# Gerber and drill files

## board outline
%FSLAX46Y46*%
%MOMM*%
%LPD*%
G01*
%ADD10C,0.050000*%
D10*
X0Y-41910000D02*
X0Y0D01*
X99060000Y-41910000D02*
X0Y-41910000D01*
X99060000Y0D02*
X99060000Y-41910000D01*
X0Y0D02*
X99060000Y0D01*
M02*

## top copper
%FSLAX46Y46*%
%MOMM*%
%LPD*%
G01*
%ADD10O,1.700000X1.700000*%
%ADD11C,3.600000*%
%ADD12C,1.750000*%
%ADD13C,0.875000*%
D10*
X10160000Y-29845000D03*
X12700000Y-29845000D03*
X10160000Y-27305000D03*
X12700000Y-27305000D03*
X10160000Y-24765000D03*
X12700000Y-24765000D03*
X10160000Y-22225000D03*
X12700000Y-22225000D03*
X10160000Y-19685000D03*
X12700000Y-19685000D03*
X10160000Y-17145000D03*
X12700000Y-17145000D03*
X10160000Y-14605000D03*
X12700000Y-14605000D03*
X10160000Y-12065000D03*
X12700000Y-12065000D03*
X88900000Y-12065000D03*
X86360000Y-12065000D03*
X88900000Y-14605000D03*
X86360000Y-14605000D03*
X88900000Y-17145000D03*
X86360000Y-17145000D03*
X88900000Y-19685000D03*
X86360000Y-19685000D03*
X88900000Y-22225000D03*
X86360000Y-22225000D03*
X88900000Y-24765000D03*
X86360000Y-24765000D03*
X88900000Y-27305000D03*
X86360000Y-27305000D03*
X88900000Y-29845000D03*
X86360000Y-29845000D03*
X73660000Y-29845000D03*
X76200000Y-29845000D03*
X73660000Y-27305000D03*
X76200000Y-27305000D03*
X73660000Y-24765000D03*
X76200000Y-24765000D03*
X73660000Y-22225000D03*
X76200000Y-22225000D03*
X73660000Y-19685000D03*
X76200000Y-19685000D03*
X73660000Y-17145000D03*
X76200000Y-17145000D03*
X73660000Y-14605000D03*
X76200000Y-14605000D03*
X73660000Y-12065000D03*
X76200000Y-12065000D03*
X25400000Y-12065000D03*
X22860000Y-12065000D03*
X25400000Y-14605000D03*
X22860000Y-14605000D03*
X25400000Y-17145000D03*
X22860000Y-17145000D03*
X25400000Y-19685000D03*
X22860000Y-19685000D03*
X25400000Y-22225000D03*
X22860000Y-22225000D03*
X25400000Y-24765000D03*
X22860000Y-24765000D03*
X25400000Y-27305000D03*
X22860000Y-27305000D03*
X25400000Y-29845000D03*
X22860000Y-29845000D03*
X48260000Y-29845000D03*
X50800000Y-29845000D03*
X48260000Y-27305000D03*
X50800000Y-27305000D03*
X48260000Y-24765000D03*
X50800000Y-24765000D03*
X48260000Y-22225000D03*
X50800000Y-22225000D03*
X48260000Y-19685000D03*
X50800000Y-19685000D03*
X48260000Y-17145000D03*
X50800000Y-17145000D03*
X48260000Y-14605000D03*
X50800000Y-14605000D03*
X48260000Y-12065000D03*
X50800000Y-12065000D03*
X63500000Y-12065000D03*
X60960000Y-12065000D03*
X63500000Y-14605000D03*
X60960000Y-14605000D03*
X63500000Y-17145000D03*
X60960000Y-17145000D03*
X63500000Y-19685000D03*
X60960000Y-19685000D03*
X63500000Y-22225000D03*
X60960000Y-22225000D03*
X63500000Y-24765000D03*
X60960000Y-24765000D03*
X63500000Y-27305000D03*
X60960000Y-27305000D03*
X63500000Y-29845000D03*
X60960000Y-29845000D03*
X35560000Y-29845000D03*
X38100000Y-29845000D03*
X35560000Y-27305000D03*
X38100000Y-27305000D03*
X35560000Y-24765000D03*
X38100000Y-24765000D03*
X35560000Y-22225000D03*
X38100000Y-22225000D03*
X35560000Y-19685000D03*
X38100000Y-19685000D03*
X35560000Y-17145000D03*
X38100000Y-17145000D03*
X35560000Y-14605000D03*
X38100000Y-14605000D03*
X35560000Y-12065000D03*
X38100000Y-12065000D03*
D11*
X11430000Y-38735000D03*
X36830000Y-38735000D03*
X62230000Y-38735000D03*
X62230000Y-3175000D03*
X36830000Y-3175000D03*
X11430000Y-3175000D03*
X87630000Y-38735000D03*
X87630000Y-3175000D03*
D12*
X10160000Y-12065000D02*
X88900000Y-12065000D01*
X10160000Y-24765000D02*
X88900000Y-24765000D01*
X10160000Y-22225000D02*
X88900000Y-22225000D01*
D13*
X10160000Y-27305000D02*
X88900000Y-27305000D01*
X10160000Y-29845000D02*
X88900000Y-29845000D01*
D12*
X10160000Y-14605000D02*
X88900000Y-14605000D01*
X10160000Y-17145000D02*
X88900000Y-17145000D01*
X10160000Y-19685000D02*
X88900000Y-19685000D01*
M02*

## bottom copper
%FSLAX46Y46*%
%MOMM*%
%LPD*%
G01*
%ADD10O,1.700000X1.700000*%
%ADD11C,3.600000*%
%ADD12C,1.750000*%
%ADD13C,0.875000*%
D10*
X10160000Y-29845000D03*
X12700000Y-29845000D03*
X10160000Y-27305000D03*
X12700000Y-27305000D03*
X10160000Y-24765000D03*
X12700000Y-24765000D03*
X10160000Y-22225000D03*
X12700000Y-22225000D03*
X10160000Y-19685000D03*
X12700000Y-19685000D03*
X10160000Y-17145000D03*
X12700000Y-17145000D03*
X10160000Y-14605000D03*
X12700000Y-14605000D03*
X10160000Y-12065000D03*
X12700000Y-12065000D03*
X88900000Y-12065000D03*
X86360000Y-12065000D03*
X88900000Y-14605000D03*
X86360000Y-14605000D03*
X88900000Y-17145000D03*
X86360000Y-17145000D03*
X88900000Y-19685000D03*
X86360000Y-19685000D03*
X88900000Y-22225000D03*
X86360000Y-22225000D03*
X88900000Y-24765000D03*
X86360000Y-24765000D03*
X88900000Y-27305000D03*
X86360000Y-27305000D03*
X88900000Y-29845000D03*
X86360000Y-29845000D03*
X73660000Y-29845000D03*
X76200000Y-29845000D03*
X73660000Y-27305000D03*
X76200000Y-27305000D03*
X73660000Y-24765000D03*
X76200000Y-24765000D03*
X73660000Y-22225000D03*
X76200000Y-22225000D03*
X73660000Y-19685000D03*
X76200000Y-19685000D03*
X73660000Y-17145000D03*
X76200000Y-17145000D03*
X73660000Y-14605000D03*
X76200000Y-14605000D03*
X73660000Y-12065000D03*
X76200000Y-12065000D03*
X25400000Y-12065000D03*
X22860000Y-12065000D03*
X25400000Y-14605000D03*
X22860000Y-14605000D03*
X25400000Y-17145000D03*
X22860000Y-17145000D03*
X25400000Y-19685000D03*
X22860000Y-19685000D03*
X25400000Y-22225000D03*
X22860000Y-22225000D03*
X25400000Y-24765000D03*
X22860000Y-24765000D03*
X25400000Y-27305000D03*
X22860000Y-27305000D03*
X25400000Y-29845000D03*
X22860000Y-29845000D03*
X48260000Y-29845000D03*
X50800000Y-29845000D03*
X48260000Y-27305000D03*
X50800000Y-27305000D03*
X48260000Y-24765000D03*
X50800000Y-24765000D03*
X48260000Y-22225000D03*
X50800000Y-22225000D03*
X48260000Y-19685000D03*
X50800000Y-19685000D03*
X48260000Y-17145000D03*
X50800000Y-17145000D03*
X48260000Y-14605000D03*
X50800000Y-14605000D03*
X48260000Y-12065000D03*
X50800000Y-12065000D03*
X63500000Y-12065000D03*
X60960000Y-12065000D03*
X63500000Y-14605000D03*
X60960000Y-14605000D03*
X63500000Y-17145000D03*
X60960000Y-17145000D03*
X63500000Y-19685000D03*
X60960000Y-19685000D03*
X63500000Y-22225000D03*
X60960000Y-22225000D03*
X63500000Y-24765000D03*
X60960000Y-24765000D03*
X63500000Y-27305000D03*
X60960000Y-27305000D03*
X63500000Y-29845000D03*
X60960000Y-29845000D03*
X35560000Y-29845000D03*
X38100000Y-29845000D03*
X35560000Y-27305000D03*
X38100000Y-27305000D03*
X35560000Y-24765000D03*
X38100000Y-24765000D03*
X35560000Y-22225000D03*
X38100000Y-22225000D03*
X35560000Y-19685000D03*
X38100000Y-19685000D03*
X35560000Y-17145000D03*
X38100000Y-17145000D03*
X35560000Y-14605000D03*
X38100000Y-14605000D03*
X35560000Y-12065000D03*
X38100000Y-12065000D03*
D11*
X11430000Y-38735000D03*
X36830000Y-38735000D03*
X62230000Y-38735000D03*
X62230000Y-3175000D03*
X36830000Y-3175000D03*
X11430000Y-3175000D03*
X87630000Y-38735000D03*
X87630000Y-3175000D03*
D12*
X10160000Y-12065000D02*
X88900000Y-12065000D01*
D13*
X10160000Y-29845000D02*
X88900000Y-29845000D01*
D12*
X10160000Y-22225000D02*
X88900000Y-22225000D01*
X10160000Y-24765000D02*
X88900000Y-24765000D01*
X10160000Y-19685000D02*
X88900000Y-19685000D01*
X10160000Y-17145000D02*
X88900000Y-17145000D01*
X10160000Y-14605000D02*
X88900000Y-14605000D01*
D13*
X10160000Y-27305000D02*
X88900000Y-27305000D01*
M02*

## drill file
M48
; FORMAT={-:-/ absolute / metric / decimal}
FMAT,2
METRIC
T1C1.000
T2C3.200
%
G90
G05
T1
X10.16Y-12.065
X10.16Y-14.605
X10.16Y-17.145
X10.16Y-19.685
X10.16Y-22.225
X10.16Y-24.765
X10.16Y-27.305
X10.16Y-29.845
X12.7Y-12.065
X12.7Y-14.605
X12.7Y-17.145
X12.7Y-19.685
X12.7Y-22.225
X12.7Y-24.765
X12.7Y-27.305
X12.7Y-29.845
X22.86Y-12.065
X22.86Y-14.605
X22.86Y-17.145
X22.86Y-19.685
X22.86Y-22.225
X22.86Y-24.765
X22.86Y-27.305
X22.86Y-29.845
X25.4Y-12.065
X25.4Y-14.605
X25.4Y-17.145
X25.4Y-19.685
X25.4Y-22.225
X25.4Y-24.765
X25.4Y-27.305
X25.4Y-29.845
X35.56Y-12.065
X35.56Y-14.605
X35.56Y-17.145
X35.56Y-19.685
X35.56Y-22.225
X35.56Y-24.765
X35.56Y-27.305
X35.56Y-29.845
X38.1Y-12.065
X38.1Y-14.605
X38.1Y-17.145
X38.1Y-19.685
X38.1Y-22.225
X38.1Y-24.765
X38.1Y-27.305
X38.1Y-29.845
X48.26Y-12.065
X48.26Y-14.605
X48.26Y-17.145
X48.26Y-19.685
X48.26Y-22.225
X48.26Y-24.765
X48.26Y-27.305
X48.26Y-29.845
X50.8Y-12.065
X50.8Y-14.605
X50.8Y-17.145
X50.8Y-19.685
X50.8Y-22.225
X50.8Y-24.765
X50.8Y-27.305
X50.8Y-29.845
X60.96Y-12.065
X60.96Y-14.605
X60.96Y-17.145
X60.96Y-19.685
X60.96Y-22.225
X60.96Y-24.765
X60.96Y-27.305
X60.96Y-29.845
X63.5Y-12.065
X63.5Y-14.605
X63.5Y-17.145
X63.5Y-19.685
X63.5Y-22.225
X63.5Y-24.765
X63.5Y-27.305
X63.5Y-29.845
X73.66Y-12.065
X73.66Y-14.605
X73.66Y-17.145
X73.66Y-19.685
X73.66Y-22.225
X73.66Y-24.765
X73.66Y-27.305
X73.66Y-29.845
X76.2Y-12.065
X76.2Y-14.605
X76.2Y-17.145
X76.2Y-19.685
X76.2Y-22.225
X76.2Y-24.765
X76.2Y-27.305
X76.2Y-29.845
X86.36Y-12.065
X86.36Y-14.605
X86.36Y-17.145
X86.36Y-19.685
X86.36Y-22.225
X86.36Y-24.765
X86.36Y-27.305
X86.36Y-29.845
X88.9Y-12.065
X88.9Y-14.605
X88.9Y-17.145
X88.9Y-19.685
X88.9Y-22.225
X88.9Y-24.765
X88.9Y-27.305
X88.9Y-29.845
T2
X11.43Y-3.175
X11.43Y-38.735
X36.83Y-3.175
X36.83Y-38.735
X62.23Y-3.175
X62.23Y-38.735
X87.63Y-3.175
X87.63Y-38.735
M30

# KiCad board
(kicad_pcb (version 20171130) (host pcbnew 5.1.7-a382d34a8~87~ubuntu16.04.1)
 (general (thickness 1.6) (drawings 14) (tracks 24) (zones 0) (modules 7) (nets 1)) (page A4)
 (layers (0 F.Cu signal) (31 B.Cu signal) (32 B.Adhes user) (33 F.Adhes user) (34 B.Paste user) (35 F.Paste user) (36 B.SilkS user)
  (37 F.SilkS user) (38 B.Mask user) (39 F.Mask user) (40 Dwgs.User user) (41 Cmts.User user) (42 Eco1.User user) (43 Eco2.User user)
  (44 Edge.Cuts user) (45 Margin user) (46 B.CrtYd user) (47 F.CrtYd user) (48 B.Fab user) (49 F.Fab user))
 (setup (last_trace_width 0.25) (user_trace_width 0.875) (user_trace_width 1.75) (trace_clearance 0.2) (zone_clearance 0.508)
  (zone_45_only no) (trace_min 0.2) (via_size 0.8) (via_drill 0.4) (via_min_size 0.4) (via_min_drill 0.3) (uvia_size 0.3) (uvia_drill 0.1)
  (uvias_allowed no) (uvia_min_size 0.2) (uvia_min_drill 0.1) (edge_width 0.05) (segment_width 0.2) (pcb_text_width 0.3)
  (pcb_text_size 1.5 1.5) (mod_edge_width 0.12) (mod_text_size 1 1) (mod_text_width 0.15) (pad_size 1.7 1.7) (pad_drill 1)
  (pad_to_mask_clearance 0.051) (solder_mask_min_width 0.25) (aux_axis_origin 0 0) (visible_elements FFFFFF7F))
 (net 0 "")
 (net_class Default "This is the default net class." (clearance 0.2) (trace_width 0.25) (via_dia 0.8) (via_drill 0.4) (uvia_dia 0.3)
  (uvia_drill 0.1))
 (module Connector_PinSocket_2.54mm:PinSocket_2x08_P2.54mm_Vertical (layer F.Cu) (at 12.7 12.065)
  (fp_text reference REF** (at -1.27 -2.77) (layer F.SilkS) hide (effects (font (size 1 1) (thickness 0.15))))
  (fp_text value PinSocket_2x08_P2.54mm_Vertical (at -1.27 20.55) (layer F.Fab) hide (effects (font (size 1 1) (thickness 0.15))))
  (pad 16 thru_hole oval (at -2.54 17.78) (size 1.7 1.7) (drill 1) (layers *.Cu *.Mask))
  (pad 15 thru_hole oval (at 0 17.78) (size 1.7 1.7) (drill 1) (layers *.Cu *.Mask))
  (pad 14 thru_hole oval (at -2.54 15.24) (size 1.7 1.7) (drill 1) (layers *.Cu *.Mask))
  (pad 13 thru_hole oval (at 0 15.24) (size 1.7 1.7) (drill 1) (layers *.Cu *.Mask))
  (pad 12 thru_hole oval (at -2.54 12.7) (size 1.7 1.7) (drill 1) (layers *.Cu *.Mask))
  (pad 11 thru_hole oval (at 0 12.7) (size 1.7 1.7) (drill 1) (layers *.Cu *.Mask))
  (pad 10 thru_hole oval (at -2.54 10.16) (size 1.7 1.7) (drill 1) (layers *.Cu *.Mask))
  (pad 9 thru_hole oval (at 0 10.16) (size 1.7 1.7) (drill 1) (layers *.Cu *.Mask))
  (pad 8 thru_hole oval (at -2.54 7.62) (size 1.7 1.7) (drill 1) (layers *.Cu *.Mask))
  (pad 7 thru_hole oval (at 0 7.62) (size 1.7 1.7) (drill 1) (layers *.Cu *.Mask))
  (pad 6 thru_hole oval (at -2.54 5.08) (size 1.7 1.7) (drill 1) (layers *.Cu *.Mask))
  (pad 5 thru_hole oval (at 0 5.08) (size 1.7 1.7) (drill 1) (layers *.Cu *.Mask))
  (pad 4 thru_hole oval (at -2.54 2.54) (size 1.7 1.7) (drill 1) (layers *.Cu *.Mask))
  (pad 3 thru_hole oval (at 0 2.54) (size 1.7 1.7) (drill 1) (layers *.Cu *.Mask))
  (pad 2 thru_hole oval (at -2.54 0) (size 1.7 1.7) (drill 1) (layers *.Cu *.Mask))
  (pad 1 thru_hole oval (at 0 0) (size 1.7 1.7) (drill 1) (layers *.Cu *.Mask)))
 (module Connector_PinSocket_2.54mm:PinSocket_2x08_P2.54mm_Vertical (layer F.Cu) (at 88.9 12.065)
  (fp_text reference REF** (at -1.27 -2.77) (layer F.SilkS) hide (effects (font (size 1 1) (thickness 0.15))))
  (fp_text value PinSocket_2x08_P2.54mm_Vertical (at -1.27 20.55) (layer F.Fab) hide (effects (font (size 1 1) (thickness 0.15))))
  (pad 1 thru_hole oval (at 0 0) (size 1.7 1.7) (drill 1) (layers *.Cu *.Mask))
  (pad 2 thru_hole oval (at -2.54 0) (size 1.7 1.7) (drill 1) (layers *.Cu *.Mask))
  (pad 3 thru_hole oval (at 0 2.54) (size 1.7 1.7) (drill 1) (layers *.Cu *.Mask))
  (pad 4 thru_hole oval (at -2.54 2.54) (size 1.7 1.7) (drill 1) (layers *.Cu *.Mask))
  (pad 5 thru_hole oval (at 0 5.08) (size 1.7 1.7) (drill 1) (layers *.Cu *.Mask))
  (pad 6 thru_hole oval (at -2.54 5.08) (size 1.7 1.7) (drill 1) (layers *.Cu *.Mask))
  (pad 7 thru_hole oval (at 0 7.62) (size 1.7 1.7) (drill 1) (layers *.Cu *.Mask))
  (pad 8 thru_hole oval (at -2.54 7.62) (size 1.7 1.7) (drill 1) (layers *.Cu *.Mask))
  (pad 9 thru_hole oval (at 0 10.16) (size 1.7 1.7) (drill 1) (layers *.Cu *.Mask))
  (pad 10 thru_hole oval (at -2.54 10.16) (size 1.7 1.7) (drill 1) (layers *.Cu *.Mask))
  (pad 11 thru_hole oval (at 0 12.7) (size 1.7 1.7) (drill 1) (layers *.Cu *.Mask))
  (pad 12 thru_hole oval (at -2.54 12.7) (size 1.7 1.7) (drill 1) (layers *.Cu *.Mask))
  (pad 13 thru_hole oval (at 0 15.24) (size 1.7 1.7) (drill 1) (layers *.Cu *.Mask))
  (pad 14 thru_hole oval (at -2.54 15.24) (size 1.7 1.7) (drill 1) (layers *.Cu *.Mask))
  (pad 15 thru_hole oval (at 0 17.78) (size 1.7 1.7) (drill 1) (layers *.Cu *.Mask))
  (pad 16 thru_hole oval (at -2.54 17.78) (size 1.7 1.7) (drill 1) (layers *.Cu *.Mask)))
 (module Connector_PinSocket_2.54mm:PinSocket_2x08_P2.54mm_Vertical (layer F.Cu) (at 76.2 12.065)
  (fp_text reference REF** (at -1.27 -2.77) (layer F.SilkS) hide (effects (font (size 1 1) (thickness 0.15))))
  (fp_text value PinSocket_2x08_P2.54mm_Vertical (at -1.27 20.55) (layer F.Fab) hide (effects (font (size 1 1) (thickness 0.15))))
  (pad 16 thru_hole oval (at -2.54 17.78) (size 1.7 1.7) (drill 1) (layers *.Cu *.Mask))
  (pad 15 thru_hole oval (at 0 17.78) (size 1.7 1.7) (drill 1) (layers *.Cu *.Mask))
  (pad 14 thru_hole oval (at -2.54 15.24) (size 1.7 1.7) (drill 1) (layers *.Cu *.Mask))
  (pad 13 thru_hole oval (at 0 15.24) (size 1.7 1.7) (drill 1) (layers *.Cu *.Mask))
  (pad 12 thru_hole oval (at -2.54 12.7) (size 1.7 1.7) (drill 1) (layers *.Cu *.Mask))
  (pad 11 thru_hole oval (at 0 12.7) (size 1.7 1.7) (drill 1) (layers *.Cu *.Mask))
  (pad 10 thru_hole oval (at -2.54 10.16) (size 1.7 1.7) (drill 1) (layers *.Cu *.Mask))
  (pad 9 thru_hole oval (at 0 10.16) (size 1.7 1.7) (drill 1) (layers *.Cu *.Mask))
  (pad 8 thru_hole oval (at -2.54 7.62) (size 1.7 1.7) (drill 1) (layers *.Cu *.Mask))
  (pad 7 thru_hole oval (at 0 7.62) (size 1.7 1.7) (drill 1) (layers *.Cu *.Mask))
  (pad 6 thru_hole oval (at -2.54 5.08) (size 1.7 1.7) (drill 1) (layers *.Cu *.Mask))
  (pad 5 thru_hole oval (at 0 5.08) (size 1.7 1.7) (drill 1) (layers *.Cu *.Mask))
  (pad 4 thru_hole oval (at -2.54 2.54) (size 1.7 1.7) (drill 1) (layers *.Cu *.Mask))
  (pad 3 thru_hole oval (at 0 2.54) (size 1.7 1.7) (drill 1) (layers *.Cu *.Mask))
  (pad 2 thru_hole oval (at -2.54 0) (size 1.7 1.7) (drill 1) (layers *.Cu *.Mask))
  (pad 1 thru_hole oval (at 0 0) (size 1.7 1.7) (drill 1) (layers *.Cu *.Mask)))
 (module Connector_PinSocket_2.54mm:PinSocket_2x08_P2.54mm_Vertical (layer F.Cu) (at 25.4 12.065)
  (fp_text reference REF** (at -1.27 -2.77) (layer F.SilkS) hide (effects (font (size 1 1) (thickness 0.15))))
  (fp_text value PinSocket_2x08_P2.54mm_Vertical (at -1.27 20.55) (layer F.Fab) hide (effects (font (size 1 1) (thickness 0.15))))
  (pad 1 thru_hole oval (at 0 0) (size 1.7 1.7) (drill 1) (layers *.Cu *.Mask))
  (pad 2 thru_hole oval (at -2.54 0) (size 1.7 1.7) (drill 1) (layers *.Cu *.Mask))
  (pad 3 thru_hole oval (at 0 2.54) (size 1.7 1.7) (drill 1) (layers *.Cu *.Mask))
  (pad 4 thru_hole oval (at -2.54 2.54) (size 1.7 1.7) (drill 1) (layers *.Cu *.Mask))
  (pad 5 thru_hole oval (at 0 5.08) (size 1.7 1.7) (drill 1) (layers *.Cu *.Mask))
  (pad 6 thru_hole oval (at -2.54 5.08) (size 1.7 1.7) (drill 1) (layers *.Cu *.Mask))
  (pad 7 thru_hole oval (at 0 7.62) (size 1.7 1.7) (drill 1) (layers *.Cu *.Mask))
  (pad 8 thru_hole oval (at -2.54 7.62) (size 1.7 1.7) (drill 1) (layers *.Cu *.Mask))
  (pad 9 thru_hole oval (at 0 10.16) (size 1.7 1.7) (drill 1) (layers *.Cu *.Mask))
  (pad 10 thru_hole oval (at -2.54 10.16) (size 1.7 1.7) (drill 1) (layers *.Cu *.Mask))
  (pad 11 thru_hole oval (at 0 12.7) (size 1.7 1.7) (drill 1) (layers *.Cu *.Mask))
  (pad 12 thru_hole oval (at -2.54 12.7) (size 1.7 1.7) (drill 1) (layers *.Cu *.Mask))
  (pad 13 thru_hole oval (at 0 15.24) (size 1.7 1.7) (drill 1) (layers *.Cu *.Mask))
  (pad 14 thru_hole oval (at -2.54 15.24) (size 1.7 1.7) (drill 1) (layers *.Cu *.Mask))
  (pad 15 thru_hole oval (at 0 17.78) (size 1.7 1.7) (drill 1) (layers *.Cu *.Mask))
  (pad 16 thru_hole oval (at -2.54 17.78) (size 1.7 1.7) (drill 1) (layers *.Cu *.Mask)))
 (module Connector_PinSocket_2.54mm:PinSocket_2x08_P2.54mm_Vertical (layer F.Cu) (at 50.8 12.065)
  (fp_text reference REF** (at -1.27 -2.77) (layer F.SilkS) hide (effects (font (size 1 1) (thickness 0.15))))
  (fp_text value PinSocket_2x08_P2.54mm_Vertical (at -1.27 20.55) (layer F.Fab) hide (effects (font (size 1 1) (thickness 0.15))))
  (pad 16 thru_hole oval (at -2.54 17.78) (size 1.7 1.7) (drill 1) (layers *.Cu *.Mask))
  (pad 15 thru_hole oval (at 0 17.78) (size 1.7 1.7) (drill 1) (layers *.Cu *.Mask))
  (pad 14 thru_hole oval (at -2.54 15.24) (size 1.7 1.7) (drill 1) (layers *.Cu *.Mask))
  (pad 13 thru_hole oval (at 0 15.24) (size 1.7 1.7) (drill 1) (layers *.Cu *.Mask))
  (pad 12 thru_hole oval (at -2.54 12.7) (size 1.7 1.7) (drill 1) (layers *.Cu *.Mask))
  (pad 11 thru_hole oval (at 0 12.7) (size 1.7 1.7) (drill 1) (layers *.Cu *.Mask))
  (pad 10 thru_hole oval (at -2.54 10.16) (size 1.7 1.7) (drill 1) (layers *.Cu *.Mask))
  (pad 9 thru_hole oval (at 0 10.16) (size 1.7 1.7) (drill 1) (layers *.Cu *.Mask))
  (pad 8 thru_hole oval (at -2.54 7.62) (size 1.7 1.7) (drill 1) (layers *.Cu *.Mask))
  (pad 7 thru_hole oval (at 0 7.62) (size 1.7 1.7) (drill 1) (layers *.Cu *.Mask))
  (pad 6 thru_hole oval (at -2.54 5.08) (size 1.7 1.7) (drill 1) (layers *.Cu *.Mask))
  (pad 5 thru_hole oval (at 0 5.08) (size 1.7 1.7) (drill 1) (layers *.Cu *.Mask))
  (pad 4 thru_hole oval (at -2.54 2.54) (size 1.7 1.7) (drill 1) (layers *.Cu *.Mask))
  (pad 3 thru_hole oval (at 0 2.54) (size 1.7 1.7) (drill 1) (layers *.Cu *.Mask))
  (pad 2 thru_hole oval (at -2.54 0) (size 1.7 1.7) (drill 1) (layers *.Cu *.Mask))
  (pad 1 thru_hole oval (at 0 0) (size 1.7 1.7) (drill 1) (layers *.Cu *.Mask)))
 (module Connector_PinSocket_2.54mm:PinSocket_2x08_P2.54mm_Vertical (layer F.Cu) (at 63.5 12.065)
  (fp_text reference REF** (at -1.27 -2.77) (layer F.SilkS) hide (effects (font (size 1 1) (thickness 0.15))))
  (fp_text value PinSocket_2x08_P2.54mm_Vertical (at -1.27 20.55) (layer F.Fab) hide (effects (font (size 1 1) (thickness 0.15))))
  (pad 1 thru_hole oval (at 0 0) (size 1.7 1.7) (drill 1) (layers *.Cu *.Mask))
  (pad 2 thru_hole oval (at -2.54 0) (size 1.7 1.7) (drill 1) (layers *.Cu *.Mask))
  (pad 3 thru_hole oval (at 0 2.54) (size 1.7 1.7) (drill 1) (layers *.Cu *.Mask))
  (pad 4 thru_hole oval (at -2.54 2.54) (size 1.7 1.7) (drill 1) (layers *.Cu *.Mask))
  (pad 5 thru_hole oval (at 0 5.08) (size 1.7 1.7) (drill 1) (layers *.Cu *.Mask))
  (pad 6 thru_hole oval (at -2.54 5.08) (size 1.7 1.7) (drill 1) (layers *.Cu *.Mask))
  (pad 7 thru_hole oval (at 0 7.62) (size 1.7 1.7) (drill 1) (layers *.Cu *.Mask))
  (pad 8 thru_hole oval (at -2.54 7.62) (size 1.7 1.7) (drill 1) (layers *.Cu *.Mask))
  (pad 9 thru_hole oval (at 0 10.16) (size 1.7 1.7) (drill 1) (layers *.Cu *.Mask))
  (pad 10 thru_hole oval (at -2.54 10.16) (size 1.7 1.7) (drill 1) (layers *.Cu *.Mask))
  (pad 11 thru_hole oval (at 0 12.7) (size 1.7 1.7) (drill 1) (layers *.Cu *.Mask))
  (pad 12 thru_hole oval (at -2.54 12.7) (size 1.7 1.7) (drill 1) (layers *.Cu *.Mask))
  (pad 13 thru_hole oval (at 0 15.24) (size 1.7 1.7) (drill 1) (layers *.Cu *.Mask))
  (pad 14 thru_hole oval (at -2.54 15.24) (size 1.7 1.7) (drill 1) (layers *.Cu *.Mask))
  (pad 15 thru_hole oval (at 0 17.78) (size 1.7 1.7) (drill 1) (layers *.Cu *.Mask))
  (pad 16 thru_hole oval (at -2.54 17.78) (size 1.7 1.7) (drill 1) (layers *.Cu *.Mask)))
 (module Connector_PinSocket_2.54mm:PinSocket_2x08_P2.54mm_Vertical (layer F.Cu) (at 38.1 12.065)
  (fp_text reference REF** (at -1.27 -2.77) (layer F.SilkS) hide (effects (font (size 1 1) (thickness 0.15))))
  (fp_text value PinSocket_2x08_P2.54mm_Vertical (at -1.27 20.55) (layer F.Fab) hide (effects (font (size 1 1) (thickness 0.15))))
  (pad 16 thru_hole oval (at -2.54 17.78) (size 1.7 1.7) (drill 1) (layers *.Cu *.Mask))
  (pad 15 thru_hole oval (at 0 17.78) (size 1.7 1.7) (drill 1) (layers *.Cu *.Mask))
  (pad 14 thru_hole oval (at -2.54 15.24) (size 1.7 1.7) (drill 1) (layers *.Cu *.Mask))
  (pad 13 thru_hole oval (at 0 15.24) (size 1.7 1.7) (drill 1) (layers *.Cu *.Mask))
  (pad 12 thru_hole oval (at -2.54 12.7) (size 1.7 1.7) (drill 1) (layers *.Cu *.Mask))
  (pad 11 thru_hole oval (at 0 12.7) (size 1.7 1.7) (drill 1) (layers *.Cu *.Mask))
  (pad 10 thru_hole oval (at -2.54 10.16) (size 1.7 1.7) (drill 1) (layers *.Cu *.Mask))
  (pad 9 thru_hole oval (at 0 10.16) (size 1.7 1.7) (drill 1) (layers *.Cu *.Mask))
  (pad 8 thru_hole oval (at -2.54 7.62) (size 1.7 1.7) (drill 1) (layers *.Cu *.Mask))
  (pad 7 thru_hole oval (at 0 7.62) (size 1.7 1.7) (drill 1) (layers *.Cu *.Mask))
  (pad 6 thru_hole oval (at -2.54 5.08) (size 1.7 1.7) (drill 1) (layers *.Cu *.Mask))
  (pad 5 thru_hole oval (at 0 5.08) (size 1.7 1.7) (drill 1) (layers *.Cu *.Mask))
  (pad 4 thru_hole oval (at -2.54 2.54) (size 1.7 1.7) (drill 1) (layers *.Cu *.Mask))
  (pad 3 thru_hole oval (at 0 2.54) (size 1.7 1.7) (drill 1) (layers *.Cu *.Mask))
  (pad 2 thru_hole oval (at -2.54 0) (size 1.7 1.7) (drill 1) (layers *.Cu *.Mask))
  (pad 1 thru_hole oval (at 0 0) (size 1.7 1.7) (drill 1) (layers *.Cu *.Mask)))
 (gr_line (start 0 41.91) (end 0 0) (layer Edge.Cuts) (width 0.05))
 (gr_line (start 99.06 41.91) (end 0 41.91) (layer Edge.Cuts) (width 0.05))
 (gr_line (start 99.06 0) (end 99.06 41.91) (layer Edge.Cuts) (width 0.05))
 (gr_line (start 0 0) (end 99.06 0) (layer Edge.Cuts) (width 0.05))
 (via (at 11.43 38.735) (size 3.6) (drill 3.2) (layers F.Cu B.Cu) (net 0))
 (via (at 36.83 38.735) (size 3.6) (drill 3.2) (layers F.Cu B.Cu) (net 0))
 (via (at 62.23 38.735) (size 3.6) (drill 3.2) (layers F.Cu B.Cu) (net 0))
 (via (at 62.23 3.175) (size 3.6) (drill 3.2) (layers F.Cu B.Cu) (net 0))
 (via (at 36.83 3.175) (size 3.6) (drill 3.2) (layers F.Cu B.Cu) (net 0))
 (via (at 11.43 3.175) (size 3.6) (drill 3.2) (layers F.Cu B.Cu) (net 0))
 (segment (start 10.16 12.065) (end 88.9 12.065) (width 1.75) (layer F.Cu) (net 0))
 (segment (start 10.16 24.765) (end 88.9 24.765) (width 1.75) (layer F.Cu) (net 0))
 (segment (start 10.16 22.225) (end 88.9 22.225) (width 1.75) (layer F.Cu) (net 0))
 (segment (start 10.16 27.305) (end 88.9 27.305) (width 0.875) (layer F.Cu) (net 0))
 (segment (start 10.16 29.845) (end 88.9 29.845) (width 0.875) (layer F.Cu) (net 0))
 (segment (start 10.16 14.605) (end 88.9 14.605) (width 1.75) (layer F.Cu) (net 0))
 (segment (start 10.16 17.145) (end 88.9 17.145) (width 1.75) (layer F.Cu) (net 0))
 (segment (start 10.16 19.685) (end 88.9 19.685) (width 1.75) (layer F.Cu) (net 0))
 (segment (start 10.16 12.065) (end 88.9 12.065) (width 1.75) (layer B.Cu) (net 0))
 (segment (start 10.16 29.845) (end 88.9 29.845) (width 0.875) (layer B.Cu) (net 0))
 (segment (start 10.16 22.225) (end 88.9 22.225) (width 1.75) (layer B.Cu) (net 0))
 (segment (start 10.16 24.765) (end 88.9 24.765) (width 1.75) (layer B.Cu) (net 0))
 (segment (start 10.16 19.685) (end 88.9 19.685) (width 1.75) (layer B.Cu) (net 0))
 (segment (start 10.16 17.145) (end 88.9 17.145) (width 1.75) (layer B.Cu) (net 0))
 (segment (start 10.16 14.605) (end 88.9 14.605) (width 1.75) (layer B.Cu) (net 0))
 (segment (start 10.16 27.305) (end 88.9 27.305) (width 0.875) (layer B.Cu) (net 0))
 (via (at 87.63 38.735) (size 3.6) (drill 3.2) (layers F.Cu B.Cu) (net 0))
 (via (at 87.63 3.175) (size 3.6) (drill 3.2) (layers F.Cu B.Cu) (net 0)))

